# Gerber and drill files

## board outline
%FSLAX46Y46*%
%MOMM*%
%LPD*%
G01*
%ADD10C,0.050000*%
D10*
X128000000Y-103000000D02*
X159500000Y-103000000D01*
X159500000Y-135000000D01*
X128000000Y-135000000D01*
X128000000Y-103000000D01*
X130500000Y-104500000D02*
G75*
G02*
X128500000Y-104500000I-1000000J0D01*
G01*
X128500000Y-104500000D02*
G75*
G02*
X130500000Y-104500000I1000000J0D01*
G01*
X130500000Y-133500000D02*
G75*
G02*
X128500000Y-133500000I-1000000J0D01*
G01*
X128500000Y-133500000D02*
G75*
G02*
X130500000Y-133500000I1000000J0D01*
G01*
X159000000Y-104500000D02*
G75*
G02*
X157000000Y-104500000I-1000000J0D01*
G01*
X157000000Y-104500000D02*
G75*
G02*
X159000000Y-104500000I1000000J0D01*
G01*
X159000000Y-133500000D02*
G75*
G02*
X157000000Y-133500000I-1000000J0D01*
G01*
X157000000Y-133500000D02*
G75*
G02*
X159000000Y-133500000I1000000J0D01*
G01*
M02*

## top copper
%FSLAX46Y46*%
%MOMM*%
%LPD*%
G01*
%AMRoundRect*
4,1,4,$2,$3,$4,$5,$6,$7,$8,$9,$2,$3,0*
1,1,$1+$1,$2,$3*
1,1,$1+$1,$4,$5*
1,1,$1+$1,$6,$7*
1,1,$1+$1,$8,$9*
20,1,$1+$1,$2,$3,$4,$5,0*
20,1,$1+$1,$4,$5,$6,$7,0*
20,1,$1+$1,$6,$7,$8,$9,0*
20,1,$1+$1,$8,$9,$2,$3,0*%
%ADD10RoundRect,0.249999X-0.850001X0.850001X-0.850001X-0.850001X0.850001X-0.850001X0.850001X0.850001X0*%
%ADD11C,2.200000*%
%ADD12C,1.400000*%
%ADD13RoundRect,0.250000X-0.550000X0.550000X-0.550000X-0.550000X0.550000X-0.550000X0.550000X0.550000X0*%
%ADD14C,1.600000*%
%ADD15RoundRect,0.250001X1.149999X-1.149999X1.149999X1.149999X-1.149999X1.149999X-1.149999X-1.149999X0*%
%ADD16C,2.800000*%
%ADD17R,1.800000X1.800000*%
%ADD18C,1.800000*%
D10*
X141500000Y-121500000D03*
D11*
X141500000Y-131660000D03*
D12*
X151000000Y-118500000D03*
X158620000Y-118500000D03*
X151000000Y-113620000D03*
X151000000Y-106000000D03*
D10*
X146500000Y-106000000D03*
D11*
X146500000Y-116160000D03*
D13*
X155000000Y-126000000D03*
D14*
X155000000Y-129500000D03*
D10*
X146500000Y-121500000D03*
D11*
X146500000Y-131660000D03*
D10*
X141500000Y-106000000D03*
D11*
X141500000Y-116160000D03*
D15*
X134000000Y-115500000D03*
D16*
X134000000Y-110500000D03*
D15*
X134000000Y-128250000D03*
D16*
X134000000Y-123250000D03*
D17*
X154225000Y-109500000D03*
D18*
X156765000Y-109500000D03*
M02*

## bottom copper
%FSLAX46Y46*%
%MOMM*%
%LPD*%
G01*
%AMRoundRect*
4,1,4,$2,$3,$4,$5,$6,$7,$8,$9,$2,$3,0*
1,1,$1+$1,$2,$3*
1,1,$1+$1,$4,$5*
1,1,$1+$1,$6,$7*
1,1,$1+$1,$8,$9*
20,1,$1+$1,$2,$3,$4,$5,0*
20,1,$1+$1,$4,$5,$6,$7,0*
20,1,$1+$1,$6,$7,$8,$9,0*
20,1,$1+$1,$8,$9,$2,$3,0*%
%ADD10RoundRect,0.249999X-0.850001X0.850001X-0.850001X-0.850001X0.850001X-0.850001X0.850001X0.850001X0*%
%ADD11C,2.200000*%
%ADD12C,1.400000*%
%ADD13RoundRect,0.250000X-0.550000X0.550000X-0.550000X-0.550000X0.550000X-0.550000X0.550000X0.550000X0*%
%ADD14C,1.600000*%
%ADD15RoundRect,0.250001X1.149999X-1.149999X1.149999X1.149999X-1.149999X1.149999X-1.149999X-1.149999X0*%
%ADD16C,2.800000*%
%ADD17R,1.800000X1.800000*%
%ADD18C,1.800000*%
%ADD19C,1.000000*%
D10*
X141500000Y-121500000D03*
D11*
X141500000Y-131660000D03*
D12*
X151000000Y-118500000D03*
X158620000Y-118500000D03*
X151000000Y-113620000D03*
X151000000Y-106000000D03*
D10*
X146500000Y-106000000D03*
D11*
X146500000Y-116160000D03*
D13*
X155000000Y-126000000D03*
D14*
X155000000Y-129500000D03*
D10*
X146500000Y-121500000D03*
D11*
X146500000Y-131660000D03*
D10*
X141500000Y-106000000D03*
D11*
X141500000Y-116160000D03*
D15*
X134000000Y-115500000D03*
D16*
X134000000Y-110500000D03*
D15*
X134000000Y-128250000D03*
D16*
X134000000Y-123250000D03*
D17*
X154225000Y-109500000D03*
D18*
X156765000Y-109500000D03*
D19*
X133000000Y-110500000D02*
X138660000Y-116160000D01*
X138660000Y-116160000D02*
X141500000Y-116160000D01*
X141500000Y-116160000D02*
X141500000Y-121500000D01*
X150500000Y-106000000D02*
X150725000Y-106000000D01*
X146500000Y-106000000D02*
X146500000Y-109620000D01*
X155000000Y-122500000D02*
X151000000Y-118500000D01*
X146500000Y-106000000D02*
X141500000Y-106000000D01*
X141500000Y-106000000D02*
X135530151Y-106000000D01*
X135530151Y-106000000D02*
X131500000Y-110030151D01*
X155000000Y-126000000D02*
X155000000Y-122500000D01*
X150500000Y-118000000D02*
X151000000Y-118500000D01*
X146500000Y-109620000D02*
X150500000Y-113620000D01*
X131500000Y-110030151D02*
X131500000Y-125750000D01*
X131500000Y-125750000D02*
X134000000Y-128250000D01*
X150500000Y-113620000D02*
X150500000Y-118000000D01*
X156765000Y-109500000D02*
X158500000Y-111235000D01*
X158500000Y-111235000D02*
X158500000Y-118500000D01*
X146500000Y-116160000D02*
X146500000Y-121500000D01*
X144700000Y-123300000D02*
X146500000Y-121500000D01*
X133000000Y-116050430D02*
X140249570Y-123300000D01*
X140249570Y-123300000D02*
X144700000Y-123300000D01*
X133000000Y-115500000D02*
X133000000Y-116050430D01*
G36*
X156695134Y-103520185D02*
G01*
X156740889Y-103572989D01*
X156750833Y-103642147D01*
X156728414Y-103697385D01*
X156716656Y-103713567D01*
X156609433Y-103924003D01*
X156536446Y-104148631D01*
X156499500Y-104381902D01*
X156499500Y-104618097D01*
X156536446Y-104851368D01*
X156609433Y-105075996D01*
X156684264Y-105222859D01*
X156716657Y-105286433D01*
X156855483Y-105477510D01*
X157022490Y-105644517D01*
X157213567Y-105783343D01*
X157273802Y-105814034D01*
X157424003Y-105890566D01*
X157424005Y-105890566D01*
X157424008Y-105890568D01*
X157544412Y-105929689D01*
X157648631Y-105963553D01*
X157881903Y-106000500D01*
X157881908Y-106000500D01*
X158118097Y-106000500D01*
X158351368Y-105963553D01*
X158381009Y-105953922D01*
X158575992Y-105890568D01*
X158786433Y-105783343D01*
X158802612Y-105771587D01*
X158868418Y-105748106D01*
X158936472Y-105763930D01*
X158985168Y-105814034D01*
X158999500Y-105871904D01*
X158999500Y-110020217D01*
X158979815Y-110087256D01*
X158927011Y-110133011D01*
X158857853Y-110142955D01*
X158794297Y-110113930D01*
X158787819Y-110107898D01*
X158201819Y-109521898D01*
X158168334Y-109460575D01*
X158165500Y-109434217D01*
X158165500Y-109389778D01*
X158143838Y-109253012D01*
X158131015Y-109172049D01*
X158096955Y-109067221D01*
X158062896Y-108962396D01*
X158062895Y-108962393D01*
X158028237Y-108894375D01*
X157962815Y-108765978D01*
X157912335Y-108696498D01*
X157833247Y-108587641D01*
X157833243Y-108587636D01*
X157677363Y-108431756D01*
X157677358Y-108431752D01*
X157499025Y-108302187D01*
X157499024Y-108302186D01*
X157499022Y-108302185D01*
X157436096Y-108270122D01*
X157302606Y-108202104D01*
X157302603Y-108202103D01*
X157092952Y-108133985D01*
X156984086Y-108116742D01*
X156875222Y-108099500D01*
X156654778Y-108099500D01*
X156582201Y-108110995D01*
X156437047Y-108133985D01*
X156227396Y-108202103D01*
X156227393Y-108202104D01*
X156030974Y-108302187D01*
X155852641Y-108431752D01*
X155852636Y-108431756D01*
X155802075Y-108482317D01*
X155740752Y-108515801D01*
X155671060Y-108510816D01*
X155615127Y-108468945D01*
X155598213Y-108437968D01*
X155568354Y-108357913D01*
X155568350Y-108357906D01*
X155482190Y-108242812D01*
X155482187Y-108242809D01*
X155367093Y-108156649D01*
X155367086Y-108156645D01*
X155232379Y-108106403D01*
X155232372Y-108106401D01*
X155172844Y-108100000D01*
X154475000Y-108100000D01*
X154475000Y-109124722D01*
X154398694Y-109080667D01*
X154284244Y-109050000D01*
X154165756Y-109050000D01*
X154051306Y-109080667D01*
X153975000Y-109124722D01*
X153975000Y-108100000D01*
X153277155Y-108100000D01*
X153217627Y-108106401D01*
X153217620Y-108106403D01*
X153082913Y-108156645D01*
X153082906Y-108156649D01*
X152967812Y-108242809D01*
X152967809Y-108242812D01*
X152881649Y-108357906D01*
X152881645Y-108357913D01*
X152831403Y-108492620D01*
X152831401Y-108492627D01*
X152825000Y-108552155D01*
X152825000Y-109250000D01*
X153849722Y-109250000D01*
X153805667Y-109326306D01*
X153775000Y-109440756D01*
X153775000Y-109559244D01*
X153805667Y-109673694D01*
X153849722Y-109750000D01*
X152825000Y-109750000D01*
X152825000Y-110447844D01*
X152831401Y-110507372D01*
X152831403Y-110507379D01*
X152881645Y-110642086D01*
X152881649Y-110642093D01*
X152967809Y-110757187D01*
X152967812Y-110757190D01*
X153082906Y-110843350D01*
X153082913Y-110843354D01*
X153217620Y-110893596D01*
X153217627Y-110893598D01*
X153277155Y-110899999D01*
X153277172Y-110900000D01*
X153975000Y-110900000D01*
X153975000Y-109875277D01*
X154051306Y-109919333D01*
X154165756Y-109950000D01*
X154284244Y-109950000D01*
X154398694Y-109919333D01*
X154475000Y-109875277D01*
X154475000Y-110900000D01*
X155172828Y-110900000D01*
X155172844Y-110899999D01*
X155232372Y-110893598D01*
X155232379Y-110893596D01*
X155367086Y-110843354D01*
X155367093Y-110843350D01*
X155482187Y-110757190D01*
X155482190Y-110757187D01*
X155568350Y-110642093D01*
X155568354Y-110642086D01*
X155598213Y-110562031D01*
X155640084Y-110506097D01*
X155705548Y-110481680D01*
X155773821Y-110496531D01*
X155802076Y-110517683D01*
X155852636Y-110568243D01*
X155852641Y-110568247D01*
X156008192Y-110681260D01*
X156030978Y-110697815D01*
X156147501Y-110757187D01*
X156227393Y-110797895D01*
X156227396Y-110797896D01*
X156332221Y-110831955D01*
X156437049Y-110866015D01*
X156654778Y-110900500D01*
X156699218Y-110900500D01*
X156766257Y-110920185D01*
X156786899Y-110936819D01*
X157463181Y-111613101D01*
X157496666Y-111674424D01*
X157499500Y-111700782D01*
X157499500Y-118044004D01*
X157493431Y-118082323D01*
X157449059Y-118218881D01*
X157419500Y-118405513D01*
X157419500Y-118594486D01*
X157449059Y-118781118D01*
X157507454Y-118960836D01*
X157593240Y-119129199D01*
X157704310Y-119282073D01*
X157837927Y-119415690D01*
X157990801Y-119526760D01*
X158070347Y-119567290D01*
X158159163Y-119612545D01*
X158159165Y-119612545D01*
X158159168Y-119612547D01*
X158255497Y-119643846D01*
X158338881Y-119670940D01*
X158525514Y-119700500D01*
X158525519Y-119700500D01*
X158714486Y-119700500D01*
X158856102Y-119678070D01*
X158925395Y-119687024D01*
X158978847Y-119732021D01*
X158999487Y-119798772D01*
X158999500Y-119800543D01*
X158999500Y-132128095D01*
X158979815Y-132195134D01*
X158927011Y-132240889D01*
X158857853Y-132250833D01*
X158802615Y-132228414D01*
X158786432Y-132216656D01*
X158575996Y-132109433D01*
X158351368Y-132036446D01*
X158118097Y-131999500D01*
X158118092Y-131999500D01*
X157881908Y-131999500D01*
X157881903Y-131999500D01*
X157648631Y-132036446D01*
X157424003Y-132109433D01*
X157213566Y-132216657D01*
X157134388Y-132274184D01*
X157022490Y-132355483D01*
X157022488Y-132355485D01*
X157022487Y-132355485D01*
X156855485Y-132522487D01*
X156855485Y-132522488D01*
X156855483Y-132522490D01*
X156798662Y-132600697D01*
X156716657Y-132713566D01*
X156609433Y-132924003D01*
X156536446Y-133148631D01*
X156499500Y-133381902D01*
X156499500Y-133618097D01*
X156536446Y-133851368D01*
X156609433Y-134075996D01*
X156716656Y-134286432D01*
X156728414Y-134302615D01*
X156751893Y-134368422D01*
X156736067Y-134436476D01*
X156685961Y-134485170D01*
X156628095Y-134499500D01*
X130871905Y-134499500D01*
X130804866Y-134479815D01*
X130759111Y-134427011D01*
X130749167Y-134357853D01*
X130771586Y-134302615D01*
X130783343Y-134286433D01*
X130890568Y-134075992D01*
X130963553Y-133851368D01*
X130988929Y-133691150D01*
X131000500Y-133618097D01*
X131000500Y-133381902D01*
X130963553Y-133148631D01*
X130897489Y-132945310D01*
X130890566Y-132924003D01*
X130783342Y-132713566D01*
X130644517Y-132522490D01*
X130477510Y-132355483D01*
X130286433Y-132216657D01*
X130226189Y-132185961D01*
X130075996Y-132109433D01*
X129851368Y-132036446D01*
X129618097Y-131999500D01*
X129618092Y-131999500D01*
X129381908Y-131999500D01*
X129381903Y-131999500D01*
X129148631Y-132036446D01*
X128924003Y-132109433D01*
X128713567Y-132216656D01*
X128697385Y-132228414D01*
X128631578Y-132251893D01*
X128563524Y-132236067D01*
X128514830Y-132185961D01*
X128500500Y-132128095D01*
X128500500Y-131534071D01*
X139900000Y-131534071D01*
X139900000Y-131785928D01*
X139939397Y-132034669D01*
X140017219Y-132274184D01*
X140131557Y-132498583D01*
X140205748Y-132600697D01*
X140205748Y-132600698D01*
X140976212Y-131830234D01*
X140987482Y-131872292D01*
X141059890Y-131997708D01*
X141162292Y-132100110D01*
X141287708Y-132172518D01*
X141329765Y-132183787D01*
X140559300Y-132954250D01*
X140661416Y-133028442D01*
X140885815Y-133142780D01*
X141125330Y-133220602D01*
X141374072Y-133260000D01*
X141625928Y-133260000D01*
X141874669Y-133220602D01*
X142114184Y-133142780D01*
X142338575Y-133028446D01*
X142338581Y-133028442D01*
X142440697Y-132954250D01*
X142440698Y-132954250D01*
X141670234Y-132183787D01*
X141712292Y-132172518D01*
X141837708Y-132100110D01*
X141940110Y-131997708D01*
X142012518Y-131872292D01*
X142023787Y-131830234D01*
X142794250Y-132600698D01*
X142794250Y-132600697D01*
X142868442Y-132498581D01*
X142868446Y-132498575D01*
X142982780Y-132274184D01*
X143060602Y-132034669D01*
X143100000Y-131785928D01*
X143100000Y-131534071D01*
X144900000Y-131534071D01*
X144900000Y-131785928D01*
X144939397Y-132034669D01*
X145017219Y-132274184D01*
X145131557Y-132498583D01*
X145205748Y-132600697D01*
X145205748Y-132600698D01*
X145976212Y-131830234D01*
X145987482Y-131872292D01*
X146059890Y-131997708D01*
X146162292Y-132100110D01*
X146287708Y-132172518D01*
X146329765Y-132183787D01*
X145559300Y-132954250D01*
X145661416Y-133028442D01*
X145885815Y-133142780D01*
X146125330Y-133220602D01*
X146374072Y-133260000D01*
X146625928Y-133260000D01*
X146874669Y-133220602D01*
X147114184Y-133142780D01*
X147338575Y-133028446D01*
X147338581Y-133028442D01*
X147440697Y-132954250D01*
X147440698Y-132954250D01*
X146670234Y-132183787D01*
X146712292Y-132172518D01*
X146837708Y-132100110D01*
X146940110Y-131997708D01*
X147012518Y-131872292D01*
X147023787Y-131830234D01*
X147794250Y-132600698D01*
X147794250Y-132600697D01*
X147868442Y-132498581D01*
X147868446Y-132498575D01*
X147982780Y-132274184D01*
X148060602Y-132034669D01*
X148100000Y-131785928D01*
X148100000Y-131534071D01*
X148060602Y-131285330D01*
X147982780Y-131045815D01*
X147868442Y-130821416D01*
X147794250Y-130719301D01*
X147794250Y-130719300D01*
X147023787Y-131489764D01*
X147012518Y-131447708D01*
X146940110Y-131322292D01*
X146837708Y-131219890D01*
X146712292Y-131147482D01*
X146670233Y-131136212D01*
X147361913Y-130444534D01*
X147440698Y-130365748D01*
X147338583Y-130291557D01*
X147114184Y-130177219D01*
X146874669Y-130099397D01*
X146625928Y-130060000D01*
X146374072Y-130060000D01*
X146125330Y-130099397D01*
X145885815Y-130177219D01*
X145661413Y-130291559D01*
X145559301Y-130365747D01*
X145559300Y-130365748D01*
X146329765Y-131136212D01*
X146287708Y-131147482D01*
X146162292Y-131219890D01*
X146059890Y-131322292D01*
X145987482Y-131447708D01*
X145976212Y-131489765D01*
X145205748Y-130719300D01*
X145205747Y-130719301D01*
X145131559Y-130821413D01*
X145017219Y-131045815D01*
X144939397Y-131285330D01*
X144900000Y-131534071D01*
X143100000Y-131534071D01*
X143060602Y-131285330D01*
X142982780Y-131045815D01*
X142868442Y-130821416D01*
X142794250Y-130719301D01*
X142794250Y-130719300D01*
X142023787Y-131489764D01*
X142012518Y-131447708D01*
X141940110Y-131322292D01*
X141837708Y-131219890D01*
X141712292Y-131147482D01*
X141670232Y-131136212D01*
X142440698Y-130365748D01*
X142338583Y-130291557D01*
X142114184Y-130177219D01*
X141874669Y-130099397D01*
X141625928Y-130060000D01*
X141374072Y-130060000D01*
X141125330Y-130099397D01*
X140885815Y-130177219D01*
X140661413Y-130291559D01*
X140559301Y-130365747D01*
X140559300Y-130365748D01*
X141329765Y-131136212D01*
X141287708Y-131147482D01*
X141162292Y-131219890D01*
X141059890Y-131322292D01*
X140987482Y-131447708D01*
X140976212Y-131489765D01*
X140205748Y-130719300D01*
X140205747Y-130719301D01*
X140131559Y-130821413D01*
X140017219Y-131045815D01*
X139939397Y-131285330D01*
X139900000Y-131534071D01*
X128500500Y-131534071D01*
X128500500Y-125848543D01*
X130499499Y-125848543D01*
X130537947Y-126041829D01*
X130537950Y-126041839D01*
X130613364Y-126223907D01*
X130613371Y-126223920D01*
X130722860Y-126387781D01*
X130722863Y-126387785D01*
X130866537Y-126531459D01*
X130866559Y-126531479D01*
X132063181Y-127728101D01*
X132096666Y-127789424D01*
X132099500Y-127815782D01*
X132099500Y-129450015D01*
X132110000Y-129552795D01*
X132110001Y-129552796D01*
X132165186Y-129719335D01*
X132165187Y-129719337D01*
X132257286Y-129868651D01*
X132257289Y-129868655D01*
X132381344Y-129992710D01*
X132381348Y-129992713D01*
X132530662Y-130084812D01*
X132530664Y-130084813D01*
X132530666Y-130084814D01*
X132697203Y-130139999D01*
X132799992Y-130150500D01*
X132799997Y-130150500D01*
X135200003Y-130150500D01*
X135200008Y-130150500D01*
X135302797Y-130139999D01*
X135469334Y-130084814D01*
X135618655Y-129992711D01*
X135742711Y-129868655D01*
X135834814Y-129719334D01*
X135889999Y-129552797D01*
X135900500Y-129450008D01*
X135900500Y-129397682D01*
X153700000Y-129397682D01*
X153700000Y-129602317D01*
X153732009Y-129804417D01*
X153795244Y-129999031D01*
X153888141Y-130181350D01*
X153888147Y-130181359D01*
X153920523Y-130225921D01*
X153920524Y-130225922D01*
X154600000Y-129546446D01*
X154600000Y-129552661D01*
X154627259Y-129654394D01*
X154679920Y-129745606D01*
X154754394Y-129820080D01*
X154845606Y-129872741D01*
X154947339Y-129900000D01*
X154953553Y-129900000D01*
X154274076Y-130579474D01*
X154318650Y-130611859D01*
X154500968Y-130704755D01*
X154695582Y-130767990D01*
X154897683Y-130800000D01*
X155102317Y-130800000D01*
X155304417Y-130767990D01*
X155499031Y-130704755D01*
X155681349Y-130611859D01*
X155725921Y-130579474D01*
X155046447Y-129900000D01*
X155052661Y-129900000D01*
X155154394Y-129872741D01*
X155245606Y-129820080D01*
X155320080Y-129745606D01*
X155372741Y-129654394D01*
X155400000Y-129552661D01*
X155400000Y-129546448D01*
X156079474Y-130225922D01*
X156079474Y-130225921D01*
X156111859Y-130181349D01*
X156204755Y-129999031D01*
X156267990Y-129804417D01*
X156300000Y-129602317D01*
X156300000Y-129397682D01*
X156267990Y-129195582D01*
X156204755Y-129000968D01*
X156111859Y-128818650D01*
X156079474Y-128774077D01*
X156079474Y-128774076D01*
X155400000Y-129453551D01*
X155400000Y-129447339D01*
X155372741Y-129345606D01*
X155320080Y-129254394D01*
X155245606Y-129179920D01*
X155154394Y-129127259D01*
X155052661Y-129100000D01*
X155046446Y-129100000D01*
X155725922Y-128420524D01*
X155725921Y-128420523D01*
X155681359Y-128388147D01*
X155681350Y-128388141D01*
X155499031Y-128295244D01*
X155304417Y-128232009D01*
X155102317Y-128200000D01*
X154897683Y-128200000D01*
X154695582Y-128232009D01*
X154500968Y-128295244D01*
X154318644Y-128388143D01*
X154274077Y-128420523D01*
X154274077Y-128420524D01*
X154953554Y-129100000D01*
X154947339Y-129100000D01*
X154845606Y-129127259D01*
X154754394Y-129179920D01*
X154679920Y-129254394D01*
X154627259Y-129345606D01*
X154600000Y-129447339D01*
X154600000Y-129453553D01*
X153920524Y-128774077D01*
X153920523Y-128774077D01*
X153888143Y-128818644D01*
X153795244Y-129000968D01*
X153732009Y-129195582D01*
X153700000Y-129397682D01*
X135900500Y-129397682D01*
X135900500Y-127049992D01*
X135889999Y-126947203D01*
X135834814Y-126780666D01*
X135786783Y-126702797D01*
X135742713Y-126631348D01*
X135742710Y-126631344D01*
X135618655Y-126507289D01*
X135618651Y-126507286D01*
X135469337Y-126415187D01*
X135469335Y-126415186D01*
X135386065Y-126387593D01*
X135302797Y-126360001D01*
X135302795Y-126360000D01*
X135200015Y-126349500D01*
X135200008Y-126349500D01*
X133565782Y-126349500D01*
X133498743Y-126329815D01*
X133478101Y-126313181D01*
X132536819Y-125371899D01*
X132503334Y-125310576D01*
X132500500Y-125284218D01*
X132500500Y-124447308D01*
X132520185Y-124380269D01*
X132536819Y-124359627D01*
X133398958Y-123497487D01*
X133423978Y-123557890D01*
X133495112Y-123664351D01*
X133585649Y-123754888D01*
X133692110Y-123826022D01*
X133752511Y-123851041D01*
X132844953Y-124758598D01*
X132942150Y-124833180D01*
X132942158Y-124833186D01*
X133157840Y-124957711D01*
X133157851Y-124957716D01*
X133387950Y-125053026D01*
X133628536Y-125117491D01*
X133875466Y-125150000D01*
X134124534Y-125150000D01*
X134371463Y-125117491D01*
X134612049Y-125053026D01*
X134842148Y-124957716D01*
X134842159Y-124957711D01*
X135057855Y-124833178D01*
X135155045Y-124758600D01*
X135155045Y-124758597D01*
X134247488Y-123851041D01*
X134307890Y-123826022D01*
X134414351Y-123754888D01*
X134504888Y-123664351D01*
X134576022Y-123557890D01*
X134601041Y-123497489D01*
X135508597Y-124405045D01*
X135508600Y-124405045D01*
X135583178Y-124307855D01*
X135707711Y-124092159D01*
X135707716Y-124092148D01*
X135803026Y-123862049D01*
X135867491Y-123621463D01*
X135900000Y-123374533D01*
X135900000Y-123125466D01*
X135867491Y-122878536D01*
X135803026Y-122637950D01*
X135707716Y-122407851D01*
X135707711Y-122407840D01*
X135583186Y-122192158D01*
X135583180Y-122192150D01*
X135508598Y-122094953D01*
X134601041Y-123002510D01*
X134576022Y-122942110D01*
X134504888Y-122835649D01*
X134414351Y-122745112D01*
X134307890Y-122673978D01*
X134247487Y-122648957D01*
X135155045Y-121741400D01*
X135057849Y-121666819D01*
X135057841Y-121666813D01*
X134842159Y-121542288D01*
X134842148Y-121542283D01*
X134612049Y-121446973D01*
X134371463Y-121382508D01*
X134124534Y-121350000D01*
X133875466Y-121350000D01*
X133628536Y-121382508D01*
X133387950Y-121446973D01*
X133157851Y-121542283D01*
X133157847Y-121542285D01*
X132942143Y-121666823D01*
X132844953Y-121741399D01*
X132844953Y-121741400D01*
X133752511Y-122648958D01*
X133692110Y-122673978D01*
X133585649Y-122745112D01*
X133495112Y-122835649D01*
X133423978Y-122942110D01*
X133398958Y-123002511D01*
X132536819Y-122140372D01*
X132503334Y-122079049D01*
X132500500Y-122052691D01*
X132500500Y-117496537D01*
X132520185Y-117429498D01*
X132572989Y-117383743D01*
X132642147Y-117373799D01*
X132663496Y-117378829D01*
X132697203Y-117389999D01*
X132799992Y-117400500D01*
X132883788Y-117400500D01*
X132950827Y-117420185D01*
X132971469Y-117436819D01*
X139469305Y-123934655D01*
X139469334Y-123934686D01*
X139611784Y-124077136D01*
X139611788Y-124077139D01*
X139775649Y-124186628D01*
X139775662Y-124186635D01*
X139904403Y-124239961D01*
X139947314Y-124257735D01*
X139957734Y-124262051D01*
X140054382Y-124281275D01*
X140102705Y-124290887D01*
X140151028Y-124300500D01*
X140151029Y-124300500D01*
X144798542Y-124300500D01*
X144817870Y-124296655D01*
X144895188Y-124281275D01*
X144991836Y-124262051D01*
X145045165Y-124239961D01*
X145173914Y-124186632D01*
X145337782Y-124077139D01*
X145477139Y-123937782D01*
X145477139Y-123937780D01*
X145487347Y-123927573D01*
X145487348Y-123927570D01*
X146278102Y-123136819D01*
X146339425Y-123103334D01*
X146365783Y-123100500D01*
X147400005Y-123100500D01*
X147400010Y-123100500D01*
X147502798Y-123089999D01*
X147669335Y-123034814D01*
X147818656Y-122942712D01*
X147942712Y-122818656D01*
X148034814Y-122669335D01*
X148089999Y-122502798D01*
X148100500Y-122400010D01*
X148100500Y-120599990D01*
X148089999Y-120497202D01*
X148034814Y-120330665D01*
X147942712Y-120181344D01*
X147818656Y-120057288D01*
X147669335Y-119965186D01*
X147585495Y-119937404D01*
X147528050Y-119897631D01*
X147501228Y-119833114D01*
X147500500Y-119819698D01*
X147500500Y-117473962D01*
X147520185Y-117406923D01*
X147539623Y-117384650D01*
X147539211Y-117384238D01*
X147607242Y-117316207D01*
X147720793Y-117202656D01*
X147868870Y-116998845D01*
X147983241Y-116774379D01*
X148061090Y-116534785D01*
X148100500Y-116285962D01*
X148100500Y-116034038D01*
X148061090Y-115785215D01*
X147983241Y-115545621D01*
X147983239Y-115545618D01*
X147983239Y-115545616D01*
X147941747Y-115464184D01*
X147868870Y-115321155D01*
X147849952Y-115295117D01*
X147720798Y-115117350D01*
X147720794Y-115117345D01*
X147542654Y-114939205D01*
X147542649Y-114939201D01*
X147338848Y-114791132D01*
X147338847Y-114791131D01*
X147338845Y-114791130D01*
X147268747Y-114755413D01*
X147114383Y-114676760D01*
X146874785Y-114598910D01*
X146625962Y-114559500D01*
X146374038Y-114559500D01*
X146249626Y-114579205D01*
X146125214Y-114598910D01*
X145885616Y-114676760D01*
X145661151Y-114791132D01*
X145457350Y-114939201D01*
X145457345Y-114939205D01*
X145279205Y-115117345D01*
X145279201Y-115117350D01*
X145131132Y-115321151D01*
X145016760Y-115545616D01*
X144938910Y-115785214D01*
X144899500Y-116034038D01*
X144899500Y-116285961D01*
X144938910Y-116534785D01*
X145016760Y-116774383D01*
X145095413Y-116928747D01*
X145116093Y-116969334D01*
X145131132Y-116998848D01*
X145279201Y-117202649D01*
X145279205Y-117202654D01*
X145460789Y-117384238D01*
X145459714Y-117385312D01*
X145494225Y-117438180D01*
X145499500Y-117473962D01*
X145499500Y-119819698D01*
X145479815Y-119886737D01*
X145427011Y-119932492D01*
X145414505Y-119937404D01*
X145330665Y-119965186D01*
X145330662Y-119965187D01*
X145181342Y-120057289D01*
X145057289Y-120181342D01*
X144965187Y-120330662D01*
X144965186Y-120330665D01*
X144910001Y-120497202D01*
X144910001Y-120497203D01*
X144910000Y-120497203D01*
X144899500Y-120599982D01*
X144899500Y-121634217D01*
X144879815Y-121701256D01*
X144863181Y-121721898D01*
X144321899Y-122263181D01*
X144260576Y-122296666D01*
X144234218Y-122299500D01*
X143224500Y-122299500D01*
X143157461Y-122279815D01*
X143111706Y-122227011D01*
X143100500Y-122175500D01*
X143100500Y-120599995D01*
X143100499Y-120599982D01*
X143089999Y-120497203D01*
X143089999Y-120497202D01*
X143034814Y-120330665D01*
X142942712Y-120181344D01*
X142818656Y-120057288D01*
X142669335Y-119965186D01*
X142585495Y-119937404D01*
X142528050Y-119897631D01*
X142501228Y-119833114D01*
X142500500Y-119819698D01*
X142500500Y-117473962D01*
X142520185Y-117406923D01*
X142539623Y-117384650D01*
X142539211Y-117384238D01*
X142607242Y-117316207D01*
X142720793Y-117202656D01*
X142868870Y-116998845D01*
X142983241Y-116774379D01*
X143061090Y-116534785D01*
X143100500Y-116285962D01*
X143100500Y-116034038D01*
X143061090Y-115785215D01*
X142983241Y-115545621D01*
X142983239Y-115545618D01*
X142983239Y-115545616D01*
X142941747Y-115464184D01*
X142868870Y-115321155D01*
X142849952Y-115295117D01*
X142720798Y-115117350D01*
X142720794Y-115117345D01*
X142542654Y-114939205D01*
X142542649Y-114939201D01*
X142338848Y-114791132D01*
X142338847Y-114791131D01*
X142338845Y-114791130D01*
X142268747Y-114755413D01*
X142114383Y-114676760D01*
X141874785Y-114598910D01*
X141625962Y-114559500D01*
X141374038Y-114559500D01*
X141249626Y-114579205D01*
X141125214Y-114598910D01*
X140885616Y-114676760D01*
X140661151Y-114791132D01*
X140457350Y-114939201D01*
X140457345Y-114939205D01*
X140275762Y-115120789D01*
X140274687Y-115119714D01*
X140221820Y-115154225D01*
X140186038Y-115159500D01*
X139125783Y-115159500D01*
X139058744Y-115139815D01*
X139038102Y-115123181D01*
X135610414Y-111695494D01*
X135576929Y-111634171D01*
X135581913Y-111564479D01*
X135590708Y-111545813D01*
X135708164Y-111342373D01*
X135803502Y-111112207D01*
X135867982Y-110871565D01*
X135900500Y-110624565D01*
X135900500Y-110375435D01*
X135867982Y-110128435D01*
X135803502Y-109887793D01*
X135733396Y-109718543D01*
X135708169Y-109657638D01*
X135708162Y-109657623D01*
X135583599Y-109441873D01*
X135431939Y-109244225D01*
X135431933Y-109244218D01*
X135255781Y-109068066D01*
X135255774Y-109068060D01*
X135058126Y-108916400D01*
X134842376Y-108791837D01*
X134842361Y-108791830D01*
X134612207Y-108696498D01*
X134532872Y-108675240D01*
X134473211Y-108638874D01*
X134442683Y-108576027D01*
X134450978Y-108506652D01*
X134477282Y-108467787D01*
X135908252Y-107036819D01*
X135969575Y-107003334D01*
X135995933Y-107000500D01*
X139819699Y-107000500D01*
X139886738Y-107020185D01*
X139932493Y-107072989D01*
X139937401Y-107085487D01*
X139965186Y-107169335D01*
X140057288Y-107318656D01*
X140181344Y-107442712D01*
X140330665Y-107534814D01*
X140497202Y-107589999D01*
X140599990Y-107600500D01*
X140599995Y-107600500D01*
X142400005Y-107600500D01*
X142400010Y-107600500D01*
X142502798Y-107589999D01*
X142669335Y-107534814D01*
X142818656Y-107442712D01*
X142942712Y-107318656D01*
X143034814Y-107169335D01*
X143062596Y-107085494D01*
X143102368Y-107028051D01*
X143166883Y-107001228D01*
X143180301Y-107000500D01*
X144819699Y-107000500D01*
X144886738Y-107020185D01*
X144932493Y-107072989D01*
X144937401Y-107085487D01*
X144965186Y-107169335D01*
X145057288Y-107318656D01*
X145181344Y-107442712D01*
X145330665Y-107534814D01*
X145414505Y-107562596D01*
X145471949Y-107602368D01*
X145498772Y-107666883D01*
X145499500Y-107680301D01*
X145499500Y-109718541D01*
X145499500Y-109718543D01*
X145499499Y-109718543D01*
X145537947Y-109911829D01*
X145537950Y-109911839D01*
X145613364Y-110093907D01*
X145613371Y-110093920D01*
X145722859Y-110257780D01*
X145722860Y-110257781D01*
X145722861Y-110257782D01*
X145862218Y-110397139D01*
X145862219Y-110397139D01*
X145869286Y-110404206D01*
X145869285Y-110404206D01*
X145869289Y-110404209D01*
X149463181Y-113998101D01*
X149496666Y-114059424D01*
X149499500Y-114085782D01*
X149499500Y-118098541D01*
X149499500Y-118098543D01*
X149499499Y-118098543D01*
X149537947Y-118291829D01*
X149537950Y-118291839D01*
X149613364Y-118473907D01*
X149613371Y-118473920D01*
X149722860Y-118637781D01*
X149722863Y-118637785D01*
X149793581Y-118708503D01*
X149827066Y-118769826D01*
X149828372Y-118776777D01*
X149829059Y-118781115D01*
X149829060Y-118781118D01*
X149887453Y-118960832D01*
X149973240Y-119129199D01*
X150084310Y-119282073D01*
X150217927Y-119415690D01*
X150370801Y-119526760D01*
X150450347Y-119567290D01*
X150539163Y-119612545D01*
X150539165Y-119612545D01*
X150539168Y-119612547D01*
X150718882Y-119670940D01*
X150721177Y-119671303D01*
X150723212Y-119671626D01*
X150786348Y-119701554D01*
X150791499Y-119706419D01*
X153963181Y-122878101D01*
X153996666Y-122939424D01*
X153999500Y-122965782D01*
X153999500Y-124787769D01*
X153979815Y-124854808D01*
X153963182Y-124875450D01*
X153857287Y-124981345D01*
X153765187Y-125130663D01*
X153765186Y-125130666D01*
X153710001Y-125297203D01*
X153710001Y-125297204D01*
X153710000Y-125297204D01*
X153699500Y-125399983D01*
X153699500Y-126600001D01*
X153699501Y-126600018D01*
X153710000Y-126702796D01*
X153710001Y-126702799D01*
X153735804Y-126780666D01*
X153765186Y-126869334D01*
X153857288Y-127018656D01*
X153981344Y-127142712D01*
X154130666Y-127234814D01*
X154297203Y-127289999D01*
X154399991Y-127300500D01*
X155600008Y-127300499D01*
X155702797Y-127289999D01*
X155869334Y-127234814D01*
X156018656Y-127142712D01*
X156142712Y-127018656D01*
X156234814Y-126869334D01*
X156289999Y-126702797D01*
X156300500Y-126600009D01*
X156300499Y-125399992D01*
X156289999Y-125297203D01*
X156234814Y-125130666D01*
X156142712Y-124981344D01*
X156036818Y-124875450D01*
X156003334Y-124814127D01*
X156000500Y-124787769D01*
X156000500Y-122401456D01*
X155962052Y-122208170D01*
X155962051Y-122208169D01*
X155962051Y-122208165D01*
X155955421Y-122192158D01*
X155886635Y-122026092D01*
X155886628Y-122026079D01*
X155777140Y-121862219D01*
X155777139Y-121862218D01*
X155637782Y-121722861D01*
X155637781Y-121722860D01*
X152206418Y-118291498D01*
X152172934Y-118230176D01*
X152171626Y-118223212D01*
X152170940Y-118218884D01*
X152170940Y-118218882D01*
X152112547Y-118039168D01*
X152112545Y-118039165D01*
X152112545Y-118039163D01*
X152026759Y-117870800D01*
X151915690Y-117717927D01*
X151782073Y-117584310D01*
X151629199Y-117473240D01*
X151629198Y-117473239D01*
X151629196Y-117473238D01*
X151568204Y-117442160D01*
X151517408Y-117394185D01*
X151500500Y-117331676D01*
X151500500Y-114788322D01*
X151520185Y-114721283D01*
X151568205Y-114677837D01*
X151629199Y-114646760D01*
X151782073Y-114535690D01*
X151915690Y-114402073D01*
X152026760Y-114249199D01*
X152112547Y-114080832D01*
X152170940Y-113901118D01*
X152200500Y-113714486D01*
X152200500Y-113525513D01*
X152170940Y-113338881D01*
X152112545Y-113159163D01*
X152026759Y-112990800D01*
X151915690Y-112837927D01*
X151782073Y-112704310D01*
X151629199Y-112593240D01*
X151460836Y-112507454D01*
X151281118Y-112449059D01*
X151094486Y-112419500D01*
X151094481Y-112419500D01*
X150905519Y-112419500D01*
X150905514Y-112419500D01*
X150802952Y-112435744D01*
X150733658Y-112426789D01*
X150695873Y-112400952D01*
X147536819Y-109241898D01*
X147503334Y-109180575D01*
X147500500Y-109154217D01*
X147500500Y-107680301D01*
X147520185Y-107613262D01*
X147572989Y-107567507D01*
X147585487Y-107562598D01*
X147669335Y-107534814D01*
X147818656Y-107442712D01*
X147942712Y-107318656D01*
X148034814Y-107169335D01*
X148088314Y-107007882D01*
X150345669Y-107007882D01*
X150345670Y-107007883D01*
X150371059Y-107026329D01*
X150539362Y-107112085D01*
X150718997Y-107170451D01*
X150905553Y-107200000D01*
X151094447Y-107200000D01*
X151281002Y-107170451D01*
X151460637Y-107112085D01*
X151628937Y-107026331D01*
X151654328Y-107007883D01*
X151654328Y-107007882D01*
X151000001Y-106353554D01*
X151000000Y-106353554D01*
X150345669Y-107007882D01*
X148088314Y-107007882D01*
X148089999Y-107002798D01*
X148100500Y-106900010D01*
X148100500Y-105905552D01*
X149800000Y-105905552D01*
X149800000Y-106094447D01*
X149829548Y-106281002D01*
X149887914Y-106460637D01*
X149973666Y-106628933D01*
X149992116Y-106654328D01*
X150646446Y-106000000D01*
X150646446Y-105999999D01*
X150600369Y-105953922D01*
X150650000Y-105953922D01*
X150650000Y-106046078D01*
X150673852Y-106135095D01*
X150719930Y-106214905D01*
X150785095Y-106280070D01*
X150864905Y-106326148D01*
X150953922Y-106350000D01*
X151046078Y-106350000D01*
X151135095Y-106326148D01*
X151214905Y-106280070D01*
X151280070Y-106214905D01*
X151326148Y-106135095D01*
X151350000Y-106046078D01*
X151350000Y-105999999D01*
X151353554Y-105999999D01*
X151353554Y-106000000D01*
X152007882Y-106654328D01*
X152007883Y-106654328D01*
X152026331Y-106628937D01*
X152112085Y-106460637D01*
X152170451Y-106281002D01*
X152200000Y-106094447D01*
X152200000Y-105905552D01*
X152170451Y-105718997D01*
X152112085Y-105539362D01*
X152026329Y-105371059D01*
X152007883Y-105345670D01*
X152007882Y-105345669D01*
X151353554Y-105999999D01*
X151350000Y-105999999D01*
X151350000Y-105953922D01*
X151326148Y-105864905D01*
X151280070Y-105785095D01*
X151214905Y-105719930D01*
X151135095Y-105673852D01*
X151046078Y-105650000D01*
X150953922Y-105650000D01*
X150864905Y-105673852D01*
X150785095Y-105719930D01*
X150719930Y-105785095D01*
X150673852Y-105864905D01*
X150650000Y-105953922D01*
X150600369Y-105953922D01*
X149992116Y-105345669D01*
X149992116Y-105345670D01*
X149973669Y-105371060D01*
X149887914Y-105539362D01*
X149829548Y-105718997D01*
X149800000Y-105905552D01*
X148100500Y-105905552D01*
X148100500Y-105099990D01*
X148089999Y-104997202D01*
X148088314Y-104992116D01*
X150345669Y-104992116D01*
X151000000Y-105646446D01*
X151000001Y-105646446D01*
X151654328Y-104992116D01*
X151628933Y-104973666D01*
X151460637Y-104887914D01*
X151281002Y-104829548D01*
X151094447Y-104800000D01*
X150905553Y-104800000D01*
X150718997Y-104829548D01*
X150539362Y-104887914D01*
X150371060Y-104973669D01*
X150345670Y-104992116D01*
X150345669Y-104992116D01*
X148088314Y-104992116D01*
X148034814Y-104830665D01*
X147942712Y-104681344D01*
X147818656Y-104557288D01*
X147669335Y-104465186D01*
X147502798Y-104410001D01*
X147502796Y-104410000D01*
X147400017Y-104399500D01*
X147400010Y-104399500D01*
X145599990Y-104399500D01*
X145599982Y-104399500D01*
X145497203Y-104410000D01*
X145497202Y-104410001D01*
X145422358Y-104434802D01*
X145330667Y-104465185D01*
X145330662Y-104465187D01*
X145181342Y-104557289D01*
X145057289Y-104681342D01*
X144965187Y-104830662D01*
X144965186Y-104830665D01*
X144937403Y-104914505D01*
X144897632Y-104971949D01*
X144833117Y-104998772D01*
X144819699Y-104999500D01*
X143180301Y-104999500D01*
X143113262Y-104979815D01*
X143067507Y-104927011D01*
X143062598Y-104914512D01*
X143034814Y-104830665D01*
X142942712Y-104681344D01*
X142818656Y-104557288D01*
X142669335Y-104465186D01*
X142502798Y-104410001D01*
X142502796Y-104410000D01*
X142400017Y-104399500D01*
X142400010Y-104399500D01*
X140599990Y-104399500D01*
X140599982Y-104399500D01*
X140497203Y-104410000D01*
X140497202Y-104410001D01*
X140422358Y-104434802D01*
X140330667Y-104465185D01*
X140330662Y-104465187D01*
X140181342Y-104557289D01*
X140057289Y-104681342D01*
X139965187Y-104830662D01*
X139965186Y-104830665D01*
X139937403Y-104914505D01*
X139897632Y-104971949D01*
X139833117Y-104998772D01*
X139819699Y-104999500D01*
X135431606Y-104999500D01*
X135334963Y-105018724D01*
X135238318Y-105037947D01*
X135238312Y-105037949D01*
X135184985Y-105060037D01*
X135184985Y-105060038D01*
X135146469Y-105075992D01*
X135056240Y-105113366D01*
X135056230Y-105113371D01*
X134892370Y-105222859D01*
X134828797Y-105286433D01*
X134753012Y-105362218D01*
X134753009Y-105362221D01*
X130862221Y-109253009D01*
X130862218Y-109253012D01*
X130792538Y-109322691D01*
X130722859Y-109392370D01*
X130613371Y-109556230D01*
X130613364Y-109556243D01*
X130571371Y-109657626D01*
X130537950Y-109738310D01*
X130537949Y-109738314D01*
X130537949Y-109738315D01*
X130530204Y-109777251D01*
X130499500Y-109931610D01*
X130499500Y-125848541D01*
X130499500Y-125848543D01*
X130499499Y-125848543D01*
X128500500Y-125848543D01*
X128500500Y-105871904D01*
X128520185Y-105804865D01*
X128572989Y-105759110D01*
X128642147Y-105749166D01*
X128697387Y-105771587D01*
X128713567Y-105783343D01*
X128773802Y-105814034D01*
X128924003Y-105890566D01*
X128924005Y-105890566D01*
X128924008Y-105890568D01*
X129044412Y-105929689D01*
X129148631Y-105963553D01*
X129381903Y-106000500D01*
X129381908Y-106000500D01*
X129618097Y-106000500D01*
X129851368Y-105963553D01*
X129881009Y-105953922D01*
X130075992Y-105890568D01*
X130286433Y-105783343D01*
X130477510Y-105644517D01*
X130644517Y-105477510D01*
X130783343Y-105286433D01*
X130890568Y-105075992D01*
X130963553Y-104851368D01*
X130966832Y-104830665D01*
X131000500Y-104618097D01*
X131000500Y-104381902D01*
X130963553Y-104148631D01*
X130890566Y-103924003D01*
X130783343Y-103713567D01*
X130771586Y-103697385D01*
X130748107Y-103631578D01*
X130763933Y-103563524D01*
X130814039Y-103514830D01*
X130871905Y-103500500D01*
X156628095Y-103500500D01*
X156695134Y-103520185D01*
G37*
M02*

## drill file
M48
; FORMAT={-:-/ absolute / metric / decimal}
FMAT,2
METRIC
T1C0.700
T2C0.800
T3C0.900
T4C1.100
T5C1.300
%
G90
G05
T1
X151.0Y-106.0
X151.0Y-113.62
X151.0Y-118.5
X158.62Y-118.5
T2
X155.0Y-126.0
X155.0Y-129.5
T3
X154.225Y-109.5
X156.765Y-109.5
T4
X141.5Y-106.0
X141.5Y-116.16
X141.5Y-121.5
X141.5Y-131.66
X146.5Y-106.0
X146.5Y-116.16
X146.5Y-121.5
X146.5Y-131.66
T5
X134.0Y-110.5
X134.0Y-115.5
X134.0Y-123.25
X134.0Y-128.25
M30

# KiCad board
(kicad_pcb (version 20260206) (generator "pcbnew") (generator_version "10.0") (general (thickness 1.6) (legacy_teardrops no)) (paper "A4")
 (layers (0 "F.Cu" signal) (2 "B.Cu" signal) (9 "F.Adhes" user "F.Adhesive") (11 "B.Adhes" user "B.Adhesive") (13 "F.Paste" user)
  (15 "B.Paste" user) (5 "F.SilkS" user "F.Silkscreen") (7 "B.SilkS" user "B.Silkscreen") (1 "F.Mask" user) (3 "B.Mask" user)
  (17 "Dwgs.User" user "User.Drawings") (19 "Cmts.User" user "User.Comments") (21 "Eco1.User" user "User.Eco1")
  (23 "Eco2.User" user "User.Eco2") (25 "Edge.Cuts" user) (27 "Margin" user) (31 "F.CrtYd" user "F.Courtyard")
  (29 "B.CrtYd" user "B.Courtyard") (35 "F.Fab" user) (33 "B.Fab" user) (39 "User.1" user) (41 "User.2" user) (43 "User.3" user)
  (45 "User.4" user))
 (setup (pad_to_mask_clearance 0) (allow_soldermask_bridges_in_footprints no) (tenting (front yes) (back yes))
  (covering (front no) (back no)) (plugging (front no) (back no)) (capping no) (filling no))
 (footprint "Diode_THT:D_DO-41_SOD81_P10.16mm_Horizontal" (layer "F.Cu") (at 141.5 121.5 -90)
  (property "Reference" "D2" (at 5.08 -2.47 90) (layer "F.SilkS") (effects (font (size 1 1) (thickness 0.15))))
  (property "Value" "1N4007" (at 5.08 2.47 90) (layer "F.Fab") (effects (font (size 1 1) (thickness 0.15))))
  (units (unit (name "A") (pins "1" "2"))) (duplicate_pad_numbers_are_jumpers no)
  (pad "1" thru_hole roundrect (at 0 0 270) (size 2.2 2.2) (drill 1.1) (layers "*.Cu" "*.Mask") (remove_unused_layers no)
   (roundrect_rratio 0.113636) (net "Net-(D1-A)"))
  (pad "2" thru_hole circle (at 10.16 0 270) (size 2.2 2.2) (drill 1.1) (layers "*.Cu" "*.Mask") (remove_unused_layers no) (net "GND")))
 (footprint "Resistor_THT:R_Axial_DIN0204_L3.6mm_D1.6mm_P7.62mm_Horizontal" (layer "F.Cu") (at 151 118.5)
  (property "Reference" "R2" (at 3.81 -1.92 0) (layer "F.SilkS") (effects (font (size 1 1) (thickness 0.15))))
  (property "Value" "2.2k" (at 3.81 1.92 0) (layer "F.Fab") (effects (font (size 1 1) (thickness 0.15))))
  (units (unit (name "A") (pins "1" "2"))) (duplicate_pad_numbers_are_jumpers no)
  (pad "1" thru_hole circle (at 0 0) (size 1.4 1.4) (drill 0.7) (layers "*.Cu" "*.Mask") (remove_unused_layers no) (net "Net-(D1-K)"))
  (pad "2" thru_hole circle (at 7.62 0) (size 1.4 1.4) (drill 0.7) (layers "*.Cu" "*.Mask") (remove_unused_layers no) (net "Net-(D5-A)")))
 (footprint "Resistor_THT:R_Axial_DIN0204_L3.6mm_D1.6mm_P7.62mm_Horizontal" (layer "F.Cu") (at 151 113.62 90)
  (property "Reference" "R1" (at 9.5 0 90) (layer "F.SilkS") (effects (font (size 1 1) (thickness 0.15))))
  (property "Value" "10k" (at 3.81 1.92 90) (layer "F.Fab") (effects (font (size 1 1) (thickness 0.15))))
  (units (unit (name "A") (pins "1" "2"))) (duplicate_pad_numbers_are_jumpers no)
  (pad "1" thru_hole circle (at 0 0 90) (size 1.4 1.4) (drill 0.7) (layers "*.Cu" "*.Mask") (remove_unused_layers no) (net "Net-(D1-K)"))
  (pad "2" thru_hole circle (at 7.62 0 90) (size 1.4 1.4) (drill 0.7) (layers "*.Cu" "*.Mask") (remove_unused_layers no) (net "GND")))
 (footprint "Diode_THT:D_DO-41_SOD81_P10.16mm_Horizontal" (layer "F.Cu") (at 146.5 106 -90)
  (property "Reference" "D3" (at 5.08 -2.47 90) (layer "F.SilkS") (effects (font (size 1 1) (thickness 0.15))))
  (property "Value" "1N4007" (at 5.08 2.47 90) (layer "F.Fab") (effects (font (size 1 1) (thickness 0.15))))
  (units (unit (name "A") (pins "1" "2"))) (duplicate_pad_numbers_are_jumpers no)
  (pad "1" thru_hole roundrect (at 0 0 270) (size 2.2 2.2) (drill 1.1) (layers "*.Cu" "*.Mask") (remove_unused_layers no)
   (roundrect_rratio 0.113636) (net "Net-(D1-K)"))
  (pad "2" thru_hole circle (at 10.16 0 270) (size 2.2 2.2) (drill 1.1) (layers "*.Cu" "*.Mask") (remove_unused_layers no)
   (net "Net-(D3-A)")))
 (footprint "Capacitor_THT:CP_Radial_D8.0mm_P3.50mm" (layer "F.Cu") (at 155 126 -90)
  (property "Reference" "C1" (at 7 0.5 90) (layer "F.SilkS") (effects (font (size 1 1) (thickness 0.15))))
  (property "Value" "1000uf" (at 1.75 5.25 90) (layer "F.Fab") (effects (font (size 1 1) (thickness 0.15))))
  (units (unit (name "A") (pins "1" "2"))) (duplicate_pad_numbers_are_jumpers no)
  (pad "1" thru_hole roundrect (at 0 0 270) (size 1.6 1.6) (drill 0.8) (layers "*.Cu" "*.Mask") (remove_unused_layers no)
   (roundrect_rratio 0.15625) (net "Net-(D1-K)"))
  (pad "2" thru_hole circle (at 3.5 0 270) (size 1.6 1.6) (drill 0.8) (layers "*.Cu" "*.Mask") (remove_unused_layers no) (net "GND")))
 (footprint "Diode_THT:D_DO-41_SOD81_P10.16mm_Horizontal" (layer "F.Cu") (at 146.5 121.5 -90)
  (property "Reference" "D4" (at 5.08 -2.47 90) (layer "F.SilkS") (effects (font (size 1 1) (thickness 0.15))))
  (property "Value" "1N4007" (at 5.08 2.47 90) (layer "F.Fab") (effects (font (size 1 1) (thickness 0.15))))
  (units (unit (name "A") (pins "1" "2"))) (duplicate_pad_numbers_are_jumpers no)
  (pad "1" thru_hole roundrect (at 0 0 270) (size 2.2 2.2) (drill 1.1) (layers "*.Cu" "*.Mask") (remove_unused_layers no)
   (roundrect_rratio 0.113636) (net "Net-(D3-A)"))
  (pad "2" thru_hole circle (at 10.16 0 270) (size 2.2 2.2) (drill 1.1) (layers "*.Cu" "*.Mask") (remove_unused_layers no) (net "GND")))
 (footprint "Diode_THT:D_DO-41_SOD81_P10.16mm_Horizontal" (layer "F.Cu") (at 141.5 106 -90)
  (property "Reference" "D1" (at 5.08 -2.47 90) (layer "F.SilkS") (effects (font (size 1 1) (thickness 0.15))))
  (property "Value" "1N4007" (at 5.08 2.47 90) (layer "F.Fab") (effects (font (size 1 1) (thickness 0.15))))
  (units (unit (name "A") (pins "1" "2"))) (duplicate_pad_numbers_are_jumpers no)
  (pad "1" thru_hole roundrect (at 0 0 270) (size 2.2 2.2) (drill 1.1) (layers "*.Cu" "*.Mask") (remove_unused_layers no)
   (roundrect_rratio 0.113636) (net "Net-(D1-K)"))
  (pad "2" thru_hole circle (at 10.16 0 270) (size 2.2 2.2) (drill 1.1) (layers "*.Cu" "*.Mask") (remove_unused_layers no)
   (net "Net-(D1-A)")))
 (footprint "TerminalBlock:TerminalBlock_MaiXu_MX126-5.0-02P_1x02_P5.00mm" (layer "F.Cu") (at 134 115.5 90)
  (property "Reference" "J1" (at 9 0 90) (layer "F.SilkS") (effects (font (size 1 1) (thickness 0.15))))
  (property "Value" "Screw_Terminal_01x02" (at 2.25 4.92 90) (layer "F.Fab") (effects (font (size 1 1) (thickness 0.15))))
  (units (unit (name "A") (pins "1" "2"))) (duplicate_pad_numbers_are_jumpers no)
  (pad "1" thru_hole roundrect (at 0 0 90) (size 2.8 2.8) (drill 1.3) (layers "*.Cu" "*.Mask") (remove_unused_layers no)
   (roundrect_rratio 0.089286) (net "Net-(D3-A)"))
  (pad "2" thru_hole circle (at 5 0 90) (size 2.8 2.8) (drill 1.3) (layers "*.Cu" "*.Mask") (remove_unused_layers no) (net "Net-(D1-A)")))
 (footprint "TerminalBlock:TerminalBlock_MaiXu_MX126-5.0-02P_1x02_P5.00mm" (layer "F.Cu") (at 134 128.25 90)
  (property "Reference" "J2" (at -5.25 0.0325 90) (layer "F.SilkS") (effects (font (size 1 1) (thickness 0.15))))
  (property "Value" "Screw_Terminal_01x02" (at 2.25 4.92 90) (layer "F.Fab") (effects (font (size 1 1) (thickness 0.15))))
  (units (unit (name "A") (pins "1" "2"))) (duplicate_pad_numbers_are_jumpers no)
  (pad "1" thru_hole roundrect (at 0 0 90) (size 2.8 2.8) (drill 1.3) (layers "*.Cu" "*.Mask") (remove_unused_layers no)
   (roundrect_rratio 0.089286) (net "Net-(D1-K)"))
  (pad "2" thru_hole circle (at 5 0 90) (size 2.8 2.8) (drill 1.3) (layers "*.Cu" "*.Mask") (remove_unused_layers no) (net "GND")))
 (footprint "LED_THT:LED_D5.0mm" (layer "F.Cu") (at 154.225 109.5)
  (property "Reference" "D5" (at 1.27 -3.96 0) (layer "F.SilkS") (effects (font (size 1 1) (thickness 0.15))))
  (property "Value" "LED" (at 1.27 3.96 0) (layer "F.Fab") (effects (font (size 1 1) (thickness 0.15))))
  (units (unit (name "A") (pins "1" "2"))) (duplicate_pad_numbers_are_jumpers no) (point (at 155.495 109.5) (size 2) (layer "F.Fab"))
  (pad "1" thru_hole rect (at 0 0) (size 1.8 1.8) (drill 0.9) (layers "*.Cu" "*.Mask") (remove_unused_layers no) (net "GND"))
  (pad "2" thru_hole circle (at 2.54 0) (size 1.8 1.8) (drill 0.9) (layers "*.Cu" "*.Mask") (remove_unused_layers no) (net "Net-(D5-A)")))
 (gr_rect (start 128 103) (end 159.5 135) (stroke (width 0.05) (type default)) (fill no) (layer "Edge.Cuts"))
 (gr_circle (center 129.5 104.5) (end 130.5 104.5) (stroke (width 0.05) (type default)) (fill no) (layer "Edge.Cuts"))
 (gr_circle (center 129.5 133.5) (end 130.5 133.5) (stroke (width 0.05) (type default)) (fill no) (layer "Edge.Cuts"))
 (gr_circle (center 158 104.5) (end 159 104.5) (stroke (width 0.05) (type default)) (fill no) (layer "Edge.Cuts"))
 (gr_circle (center 158 133.5) (end 159 133.5) (stroke (width 0.05) (type default)) (fill no) (layer "Edge.Cuts"))
 (segment (start 133 110.5) (end 138.66 116.16) (width 1) (layer "B.Cu") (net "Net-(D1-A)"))
 (segment (start 138.66 116.16) (end 141.5 116.16) (width 1) (layer "B.Cu") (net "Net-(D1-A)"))
 (segment (start 141.5 116.16) (end 141.5 121.5) (width 1) (layer "B.Cu") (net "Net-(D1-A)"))
 (segment (start 150.5 106) (end 150.725 106) (width 1) (layer "B.Cu") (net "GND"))
 (segment (start 146.5 106) (end 146.5 109.62) (width 1) (layer "B.Cu") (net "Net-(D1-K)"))
 (segment (start 155 122.5) (end 151 118.5) (width 1) (layer "B.Cu") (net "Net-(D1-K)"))
 (segment (start 146.5 106) (end 141.5 106) (width 1) (layer "B.Cu") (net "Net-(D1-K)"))
 (segment (start 141.5 106) (end 135.530151 106) (width 1) (layer "B.Cu") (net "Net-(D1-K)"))
 (segment (start 135.530151 106) (end 131.5 110.030151) (width 1) (layer "B.Cu") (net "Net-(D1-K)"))
 (segment (start 155 126) (end 155 122.5) (width 1) (layer "B.Cu") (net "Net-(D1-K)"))
 (segment (start 150.5 118) (end 151 118.5) (width 1) (layer "B.Cu") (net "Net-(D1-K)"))
 (segment (start 146.5 109.62) (end 150.5 113.62) (width 1) (layer "B.Cu") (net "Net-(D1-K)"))
 (segment (start 131.5 110.030151) (end 131.5 125.75) (width 1) (layer "B.Cu") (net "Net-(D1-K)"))
 (segment (start 131.5 125.75) (end 134 128.25) (width 1) (layer "B.Cu") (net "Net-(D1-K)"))
 (segment (start 150.5 113.62) (end 150.5 118) (width 1) (layer "B.Cu") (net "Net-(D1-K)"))
 (segment (start 156.765 109.5) (end 158.5 111.235) (width 1) (layer "B.Cu") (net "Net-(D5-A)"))
 (segment (start 158.5 111.235) (end 158.5 118.5) (width 1) (layer "B.Cu") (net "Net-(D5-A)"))
 (segment (start 146.5 116.16) (end 146.5 121.5) (width 1) (layer "B.Cu") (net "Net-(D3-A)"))
 (segment (start 144.7 123.3) (end 146.5 121.5) (width 1) (layer "B.Cu") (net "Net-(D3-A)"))
 (segment (start 133 116.05043) (end 140.24957 123.3) (width 1) (layer "B.Cu") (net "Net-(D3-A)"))
 (segment (start 140.24957 123.3) (end 144.7 123.3) (width 1) (layer "B.Cu") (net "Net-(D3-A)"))
 (segment (start 133 115.5) (end 133 116.05043) (width 1) (layer "B.Cu") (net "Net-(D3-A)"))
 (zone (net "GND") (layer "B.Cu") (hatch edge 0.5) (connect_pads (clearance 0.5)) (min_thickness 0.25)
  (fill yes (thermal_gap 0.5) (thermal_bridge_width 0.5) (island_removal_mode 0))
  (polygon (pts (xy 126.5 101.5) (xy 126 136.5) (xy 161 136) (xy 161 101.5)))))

